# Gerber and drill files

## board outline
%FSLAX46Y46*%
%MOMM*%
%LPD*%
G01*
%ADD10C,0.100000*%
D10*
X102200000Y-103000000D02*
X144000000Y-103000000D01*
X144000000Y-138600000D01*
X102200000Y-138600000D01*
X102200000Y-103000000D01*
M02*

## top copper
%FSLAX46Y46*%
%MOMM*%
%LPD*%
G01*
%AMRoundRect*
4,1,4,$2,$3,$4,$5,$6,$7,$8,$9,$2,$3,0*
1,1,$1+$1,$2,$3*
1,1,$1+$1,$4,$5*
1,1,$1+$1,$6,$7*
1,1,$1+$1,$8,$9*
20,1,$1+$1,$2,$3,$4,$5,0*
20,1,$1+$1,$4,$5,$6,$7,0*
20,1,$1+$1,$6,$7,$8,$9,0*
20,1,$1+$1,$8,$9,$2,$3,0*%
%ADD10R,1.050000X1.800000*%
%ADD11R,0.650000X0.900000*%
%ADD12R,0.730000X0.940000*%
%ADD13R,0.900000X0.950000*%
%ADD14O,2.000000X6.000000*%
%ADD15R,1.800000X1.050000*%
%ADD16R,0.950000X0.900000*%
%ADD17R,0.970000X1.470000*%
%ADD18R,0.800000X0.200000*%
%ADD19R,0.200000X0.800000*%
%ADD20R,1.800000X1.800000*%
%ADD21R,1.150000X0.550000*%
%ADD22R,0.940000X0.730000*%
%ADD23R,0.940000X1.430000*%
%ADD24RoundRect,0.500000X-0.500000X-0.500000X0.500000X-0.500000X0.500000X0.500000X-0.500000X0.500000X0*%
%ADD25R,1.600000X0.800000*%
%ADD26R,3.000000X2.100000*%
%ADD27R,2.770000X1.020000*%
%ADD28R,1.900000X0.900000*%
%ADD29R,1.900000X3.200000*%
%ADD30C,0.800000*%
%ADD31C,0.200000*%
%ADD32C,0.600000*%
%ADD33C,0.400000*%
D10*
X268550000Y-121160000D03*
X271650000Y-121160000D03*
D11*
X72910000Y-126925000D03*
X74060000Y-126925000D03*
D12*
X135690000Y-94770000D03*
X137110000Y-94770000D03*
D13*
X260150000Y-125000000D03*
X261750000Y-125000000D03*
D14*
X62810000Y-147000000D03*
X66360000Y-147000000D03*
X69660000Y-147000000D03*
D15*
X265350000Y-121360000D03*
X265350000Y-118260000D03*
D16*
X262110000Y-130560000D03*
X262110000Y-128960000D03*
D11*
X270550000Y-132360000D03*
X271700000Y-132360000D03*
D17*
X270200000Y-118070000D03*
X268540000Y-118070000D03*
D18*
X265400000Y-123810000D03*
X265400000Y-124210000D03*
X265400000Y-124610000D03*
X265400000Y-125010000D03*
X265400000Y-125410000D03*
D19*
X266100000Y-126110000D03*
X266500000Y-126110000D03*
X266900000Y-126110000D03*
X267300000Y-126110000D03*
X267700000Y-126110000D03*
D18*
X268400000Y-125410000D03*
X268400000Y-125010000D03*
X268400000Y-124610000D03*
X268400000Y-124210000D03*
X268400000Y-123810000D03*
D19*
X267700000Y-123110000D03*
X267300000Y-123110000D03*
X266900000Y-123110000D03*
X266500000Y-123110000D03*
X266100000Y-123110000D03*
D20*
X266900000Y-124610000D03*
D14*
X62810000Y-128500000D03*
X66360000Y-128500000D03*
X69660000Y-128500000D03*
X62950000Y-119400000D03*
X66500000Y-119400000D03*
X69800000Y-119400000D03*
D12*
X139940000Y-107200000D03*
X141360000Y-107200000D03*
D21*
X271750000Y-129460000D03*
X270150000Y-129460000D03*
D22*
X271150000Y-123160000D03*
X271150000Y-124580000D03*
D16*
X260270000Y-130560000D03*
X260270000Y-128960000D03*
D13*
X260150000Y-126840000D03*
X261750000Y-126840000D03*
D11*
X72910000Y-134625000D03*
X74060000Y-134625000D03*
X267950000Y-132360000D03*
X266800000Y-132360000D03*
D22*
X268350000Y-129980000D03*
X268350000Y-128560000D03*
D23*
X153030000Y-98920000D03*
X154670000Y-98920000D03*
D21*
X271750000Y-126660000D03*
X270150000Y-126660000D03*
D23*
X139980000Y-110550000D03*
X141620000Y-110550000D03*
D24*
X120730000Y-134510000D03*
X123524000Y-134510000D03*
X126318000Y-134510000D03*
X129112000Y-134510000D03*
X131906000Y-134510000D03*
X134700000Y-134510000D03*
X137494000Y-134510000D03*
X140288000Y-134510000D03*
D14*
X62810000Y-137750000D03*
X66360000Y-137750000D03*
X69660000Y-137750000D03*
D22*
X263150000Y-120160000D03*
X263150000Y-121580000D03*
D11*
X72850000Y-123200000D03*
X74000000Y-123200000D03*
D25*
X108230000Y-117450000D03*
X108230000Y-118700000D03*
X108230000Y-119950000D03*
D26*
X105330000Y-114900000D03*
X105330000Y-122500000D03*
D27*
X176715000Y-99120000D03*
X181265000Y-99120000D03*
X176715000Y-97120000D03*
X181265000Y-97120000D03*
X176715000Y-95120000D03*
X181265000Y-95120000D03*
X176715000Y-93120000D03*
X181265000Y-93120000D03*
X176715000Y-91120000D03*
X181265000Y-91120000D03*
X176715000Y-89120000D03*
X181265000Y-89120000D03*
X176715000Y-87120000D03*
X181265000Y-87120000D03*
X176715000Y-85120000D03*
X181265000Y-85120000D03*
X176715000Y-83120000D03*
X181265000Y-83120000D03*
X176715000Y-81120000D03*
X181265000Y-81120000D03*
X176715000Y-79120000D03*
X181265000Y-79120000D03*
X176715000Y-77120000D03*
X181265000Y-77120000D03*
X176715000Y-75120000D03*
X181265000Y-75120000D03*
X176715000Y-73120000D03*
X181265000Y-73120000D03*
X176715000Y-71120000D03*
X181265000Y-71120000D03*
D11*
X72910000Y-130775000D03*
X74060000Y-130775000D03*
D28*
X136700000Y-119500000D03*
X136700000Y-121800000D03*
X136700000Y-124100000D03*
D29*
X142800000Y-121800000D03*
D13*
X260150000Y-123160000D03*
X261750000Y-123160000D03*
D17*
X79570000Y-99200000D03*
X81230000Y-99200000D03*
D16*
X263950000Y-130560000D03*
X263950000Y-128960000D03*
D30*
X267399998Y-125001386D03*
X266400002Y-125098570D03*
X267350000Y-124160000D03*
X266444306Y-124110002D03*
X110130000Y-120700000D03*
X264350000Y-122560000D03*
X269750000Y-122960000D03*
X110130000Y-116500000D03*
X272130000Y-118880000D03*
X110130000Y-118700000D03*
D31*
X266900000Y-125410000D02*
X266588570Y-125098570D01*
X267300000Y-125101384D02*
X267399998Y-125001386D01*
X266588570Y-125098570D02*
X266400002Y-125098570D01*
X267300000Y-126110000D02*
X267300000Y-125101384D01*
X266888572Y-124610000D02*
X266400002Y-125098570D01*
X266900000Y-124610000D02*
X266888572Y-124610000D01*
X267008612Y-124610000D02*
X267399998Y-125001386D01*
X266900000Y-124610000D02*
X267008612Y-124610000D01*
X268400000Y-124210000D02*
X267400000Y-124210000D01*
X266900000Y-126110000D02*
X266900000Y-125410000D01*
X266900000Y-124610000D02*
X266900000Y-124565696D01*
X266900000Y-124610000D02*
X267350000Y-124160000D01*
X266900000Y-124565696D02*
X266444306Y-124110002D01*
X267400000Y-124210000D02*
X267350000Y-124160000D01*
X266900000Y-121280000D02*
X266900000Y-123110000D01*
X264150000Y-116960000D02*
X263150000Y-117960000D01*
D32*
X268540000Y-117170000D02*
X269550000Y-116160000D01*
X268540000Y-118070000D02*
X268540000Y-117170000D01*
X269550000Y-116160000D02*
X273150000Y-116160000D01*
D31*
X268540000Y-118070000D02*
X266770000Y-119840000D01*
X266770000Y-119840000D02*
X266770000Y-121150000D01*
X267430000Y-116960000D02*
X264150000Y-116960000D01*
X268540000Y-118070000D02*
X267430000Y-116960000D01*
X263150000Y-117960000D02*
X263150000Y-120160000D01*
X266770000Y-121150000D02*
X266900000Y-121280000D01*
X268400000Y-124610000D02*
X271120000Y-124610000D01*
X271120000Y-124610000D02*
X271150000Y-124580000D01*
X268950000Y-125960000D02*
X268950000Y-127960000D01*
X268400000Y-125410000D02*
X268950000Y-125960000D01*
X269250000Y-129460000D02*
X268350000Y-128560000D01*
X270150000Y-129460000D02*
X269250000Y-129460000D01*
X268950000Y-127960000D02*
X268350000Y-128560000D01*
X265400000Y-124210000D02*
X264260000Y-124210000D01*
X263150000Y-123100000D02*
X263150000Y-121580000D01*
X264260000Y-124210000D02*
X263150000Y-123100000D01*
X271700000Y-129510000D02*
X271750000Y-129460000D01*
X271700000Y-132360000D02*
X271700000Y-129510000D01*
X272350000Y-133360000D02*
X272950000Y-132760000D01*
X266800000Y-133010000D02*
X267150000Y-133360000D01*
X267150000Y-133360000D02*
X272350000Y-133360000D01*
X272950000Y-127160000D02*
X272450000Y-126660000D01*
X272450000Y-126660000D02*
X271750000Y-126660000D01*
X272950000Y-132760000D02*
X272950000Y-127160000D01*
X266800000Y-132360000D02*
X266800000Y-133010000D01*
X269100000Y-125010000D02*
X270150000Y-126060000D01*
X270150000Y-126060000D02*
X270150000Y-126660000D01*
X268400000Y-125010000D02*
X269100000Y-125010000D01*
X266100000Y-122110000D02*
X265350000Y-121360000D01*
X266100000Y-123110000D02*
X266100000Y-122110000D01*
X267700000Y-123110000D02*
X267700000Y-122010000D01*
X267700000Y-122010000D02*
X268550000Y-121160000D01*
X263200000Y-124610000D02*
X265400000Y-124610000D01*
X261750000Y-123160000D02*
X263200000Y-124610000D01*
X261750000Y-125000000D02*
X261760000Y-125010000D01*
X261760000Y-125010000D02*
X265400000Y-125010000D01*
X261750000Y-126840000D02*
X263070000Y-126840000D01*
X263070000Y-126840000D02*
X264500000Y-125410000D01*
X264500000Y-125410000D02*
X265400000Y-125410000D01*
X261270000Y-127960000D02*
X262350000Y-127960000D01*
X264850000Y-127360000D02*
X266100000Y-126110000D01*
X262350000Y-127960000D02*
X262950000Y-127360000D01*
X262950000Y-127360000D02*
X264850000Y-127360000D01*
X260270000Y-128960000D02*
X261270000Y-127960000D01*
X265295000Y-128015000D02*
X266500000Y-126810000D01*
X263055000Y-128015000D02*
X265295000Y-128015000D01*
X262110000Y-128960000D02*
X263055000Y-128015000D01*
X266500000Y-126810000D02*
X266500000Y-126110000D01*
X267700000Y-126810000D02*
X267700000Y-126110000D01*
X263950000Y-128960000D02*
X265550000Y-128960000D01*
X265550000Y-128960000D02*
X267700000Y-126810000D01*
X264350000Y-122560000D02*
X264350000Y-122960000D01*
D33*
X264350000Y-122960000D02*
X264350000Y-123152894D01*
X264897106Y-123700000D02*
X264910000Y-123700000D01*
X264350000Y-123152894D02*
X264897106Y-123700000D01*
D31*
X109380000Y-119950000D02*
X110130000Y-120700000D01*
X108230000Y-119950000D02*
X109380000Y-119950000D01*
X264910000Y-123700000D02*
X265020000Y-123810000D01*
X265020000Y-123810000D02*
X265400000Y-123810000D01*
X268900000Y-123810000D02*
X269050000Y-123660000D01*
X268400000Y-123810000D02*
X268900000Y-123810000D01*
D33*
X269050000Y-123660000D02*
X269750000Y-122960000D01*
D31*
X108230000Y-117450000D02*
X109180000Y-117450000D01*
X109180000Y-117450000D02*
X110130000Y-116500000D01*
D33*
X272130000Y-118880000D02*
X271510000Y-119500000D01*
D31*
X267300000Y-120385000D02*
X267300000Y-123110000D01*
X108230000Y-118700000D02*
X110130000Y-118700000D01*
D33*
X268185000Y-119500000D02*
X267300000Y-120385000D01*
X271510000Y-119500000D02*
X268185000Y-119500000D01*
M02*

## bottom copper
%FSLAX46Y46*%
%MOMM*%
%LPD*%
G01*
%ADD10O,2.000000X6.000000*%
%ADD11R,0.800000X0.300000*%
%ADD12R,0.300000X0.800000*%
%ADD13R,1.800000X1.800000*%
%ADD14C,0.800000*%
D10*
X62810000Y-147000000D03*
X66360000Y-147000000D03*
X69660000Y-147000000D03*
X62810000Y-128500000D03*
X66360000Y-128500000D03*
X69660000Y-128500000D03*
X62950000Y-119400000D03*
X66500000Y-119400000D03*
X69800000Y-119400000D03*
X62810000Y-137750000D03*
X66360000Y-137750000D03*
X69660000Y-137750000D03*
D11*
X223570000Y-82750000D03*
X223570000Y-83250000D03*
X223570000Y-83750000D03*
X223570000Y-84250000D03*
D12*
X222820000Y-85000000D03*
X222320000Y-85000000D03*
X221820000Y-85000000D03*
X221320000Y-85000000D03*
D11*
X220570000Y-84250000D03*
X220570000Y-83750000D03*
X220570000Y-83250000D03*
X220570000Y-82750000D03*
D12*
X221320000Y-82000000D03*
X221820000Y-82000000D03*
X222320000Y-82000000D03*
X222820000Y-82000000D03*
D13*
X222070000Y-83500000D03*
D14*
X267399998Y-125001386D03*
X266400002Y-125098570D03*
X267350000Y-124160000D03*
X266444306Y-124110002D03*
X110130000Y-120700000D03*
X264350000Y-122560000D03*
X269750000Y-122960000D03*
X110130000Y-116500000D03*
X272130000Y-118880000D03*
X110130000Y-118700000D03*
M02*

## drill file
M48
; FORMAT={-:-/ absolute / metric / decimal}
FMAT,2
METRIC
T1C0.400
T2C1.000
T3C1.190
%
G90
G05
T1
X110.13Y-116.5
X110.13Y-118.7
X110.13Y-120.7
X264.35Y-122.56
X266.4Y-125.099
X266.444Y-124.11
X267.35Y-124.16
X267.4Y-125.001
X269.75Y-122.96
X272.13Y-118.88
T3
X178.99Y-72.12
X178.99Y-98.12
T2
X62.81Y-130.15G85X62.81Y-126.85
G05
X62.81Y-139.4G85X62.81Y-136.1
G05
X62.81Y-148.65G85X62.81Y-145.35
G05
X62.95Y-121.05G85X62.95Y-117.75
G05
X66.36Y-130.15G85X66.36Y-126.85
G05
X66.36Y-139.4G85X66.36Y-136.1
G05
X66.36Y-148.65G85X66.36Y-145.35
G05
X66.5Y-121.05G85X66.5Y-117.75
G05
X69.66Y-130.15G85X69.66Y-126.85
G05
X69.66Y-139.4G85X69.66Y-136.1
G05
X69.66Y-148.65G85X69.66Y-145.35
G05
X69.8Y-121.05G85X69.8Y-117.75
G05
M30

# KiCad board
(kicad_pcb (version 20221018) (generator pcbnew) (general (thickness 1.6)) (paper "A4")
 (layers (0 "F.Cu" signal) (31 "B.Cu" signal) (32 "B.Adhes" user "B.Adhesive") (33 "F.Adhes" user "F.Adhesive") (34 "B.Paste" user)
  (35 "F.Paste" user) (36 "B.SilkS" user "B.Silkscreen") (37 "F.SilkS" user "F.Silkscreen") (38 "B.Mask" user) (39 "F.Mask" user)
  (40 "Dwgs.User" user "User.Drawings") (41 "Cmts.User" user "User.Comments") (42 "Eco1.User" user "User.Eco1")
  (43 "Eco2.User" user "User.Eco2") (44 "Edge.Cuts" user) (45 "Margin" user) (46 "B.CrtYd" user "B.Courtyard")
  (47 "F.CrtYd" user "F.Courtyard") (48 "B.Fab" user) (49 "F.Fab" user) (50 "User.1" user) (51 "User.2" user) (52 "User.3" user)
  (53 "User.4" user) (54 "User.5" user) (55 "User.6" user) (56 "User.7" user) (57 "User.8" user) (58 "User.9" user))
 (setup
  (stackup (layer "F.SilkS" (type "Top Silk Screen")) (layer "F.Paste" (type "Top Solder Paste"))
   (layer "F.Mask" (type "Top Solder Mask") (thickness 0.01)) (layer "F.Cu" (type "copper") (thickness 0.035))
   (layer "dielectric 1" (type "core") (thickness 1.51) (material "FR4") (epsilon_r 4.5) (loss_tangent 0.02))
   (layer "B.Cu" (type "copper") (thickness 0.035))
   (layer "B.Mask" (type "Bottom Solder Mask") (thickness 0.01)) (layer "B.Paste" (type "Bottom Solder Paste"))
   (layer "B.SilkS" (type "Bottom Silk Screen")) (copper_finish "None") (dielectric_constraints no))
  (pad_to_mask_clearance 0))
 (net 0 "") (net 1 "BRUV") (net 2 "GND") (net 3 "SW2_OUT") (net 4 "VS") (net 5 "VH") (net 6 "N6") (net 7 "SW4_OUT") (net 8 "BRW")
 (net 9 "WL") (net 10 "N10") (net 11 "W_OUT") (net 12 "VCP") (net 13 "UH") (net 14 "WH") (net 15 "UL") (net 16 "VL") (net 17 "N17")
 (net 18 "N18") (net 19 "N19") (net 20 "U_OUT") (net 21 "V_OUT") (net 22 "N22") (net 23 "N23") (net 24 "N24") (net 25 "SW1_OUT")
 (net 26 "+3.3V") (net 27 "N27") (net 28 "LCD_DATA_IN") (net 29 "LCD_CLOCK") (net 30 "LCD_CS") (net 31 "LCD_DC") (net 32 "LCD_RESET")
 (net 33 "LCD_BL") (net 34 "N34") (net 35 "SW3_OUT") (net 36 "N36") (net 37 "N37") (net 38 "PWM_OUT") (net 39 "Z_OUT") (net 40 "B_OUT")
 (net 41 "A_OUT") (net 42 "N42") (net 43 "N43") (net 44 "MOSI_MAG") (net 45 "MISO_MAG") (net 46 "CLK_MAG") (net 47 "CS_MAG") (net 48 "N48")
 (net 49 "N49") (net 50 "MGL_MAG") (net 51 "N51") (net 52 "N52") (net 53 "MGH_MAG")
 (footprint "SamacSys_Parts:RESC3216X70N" (layer "F.Cu") (at 270.1 121.16)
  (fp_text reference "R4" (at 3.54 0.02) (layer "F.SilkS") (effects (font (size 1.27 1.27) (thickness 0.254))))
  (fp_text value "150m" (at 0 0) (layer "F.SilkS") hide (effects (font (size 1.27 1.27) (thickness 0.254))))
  (pad "1" smd rect (at -1.55 0) (size 1.05 1.8) (layers "F.Cu" "F.Paste" "F.Mask") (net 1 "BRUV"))
  (pad "2" smd rect (at 1.55 0) (size 1.05 1.8) (layers "F.Cu" "F.Paste" "F.Mask") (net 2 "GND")))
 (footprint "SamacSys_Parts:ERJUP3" (layer "F.Cu") (at 73.485 126.925)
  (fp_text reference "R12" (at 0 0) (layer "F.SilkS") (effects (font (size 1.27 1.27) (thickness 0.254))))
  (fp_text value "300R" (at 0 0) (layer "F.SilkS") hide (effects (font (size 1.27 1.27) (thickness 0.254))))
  (pad "1" smd rect (at -0.575 0) (size 0.65 0.9) (layers "F.Cu" "F.Paste" "F.Mask") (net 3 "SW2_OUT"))
  (pad "2" smd rect (at 0.575 0) (size 0.65 0.9) (layers "F.Cu" "F.Paste" "F.Mask") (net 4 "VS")))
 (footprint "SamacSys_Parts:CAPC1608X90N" (layer "F.Cu") (at 136.4 94.77)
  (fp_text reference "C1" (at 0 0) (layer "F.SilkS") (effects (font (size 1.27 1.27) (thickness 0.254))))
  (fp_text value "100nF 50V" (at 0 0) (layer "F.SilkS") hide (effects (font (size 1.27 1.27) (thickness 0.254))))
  (pad "1" smd rect (at -0.71 0) (size 0.73 0.94) (layers "F.Cu" "F.Paste" "F.Mask") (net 2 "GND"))
  (pad "2" smd rect (at 0.71 0) (size 0.73 0.94) (layers "F.Cu" "F.Paste" "F.Mask") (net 4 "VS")))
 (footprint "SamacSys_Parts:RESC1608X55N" (layer "F.Cu") (at 260.95 125)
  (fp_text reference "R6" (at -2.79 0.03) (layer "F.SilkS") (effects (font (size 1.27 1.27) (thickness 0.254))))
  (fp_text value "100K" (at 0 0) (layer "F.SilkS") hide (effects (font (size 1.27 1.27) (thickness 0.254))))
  (pad "1" smd rect (at -0.8 0) (size 0.9 0.95) (layers "F.Cu" "F.Paste" "F.Mask") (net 2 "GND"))
  (pad "2" smd rect (at 0.8 0) (size 0.9 0.95) (layers "F.Cu" "F.Paste" "F.Mask") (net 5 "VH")))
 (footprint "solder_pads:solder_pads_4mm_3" (layer "F.Cu") (at 66.6 152)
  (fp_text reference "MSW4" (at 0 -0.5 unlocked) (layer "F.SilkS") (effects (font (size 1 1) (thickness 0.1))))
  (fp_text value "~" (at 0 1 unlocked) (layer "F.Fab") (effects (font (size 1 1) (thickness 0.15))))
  (pad "1" thru_hole oval (at -3.79 -5 90) (size 6 2) (drill oval 4.3 1) (layers "*.Cu" "*.Mask") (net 2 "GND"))
  (pad "2" thru_hole oval (at -0.24 -5 90) (size 6 2) (drill oval 4.3 1) (layers "*.Cu" "*.Mask") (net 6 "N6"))
  (pad "4" thru_hole oval (at 3.06 -5 90) (size 6 2) (drill oval 4.3 1) (layers "*.Cu" "*.Mask") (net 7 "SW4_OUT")))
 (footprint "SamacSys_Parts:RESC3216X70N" (layer "F.Cu") (at 265.35 119.81 90)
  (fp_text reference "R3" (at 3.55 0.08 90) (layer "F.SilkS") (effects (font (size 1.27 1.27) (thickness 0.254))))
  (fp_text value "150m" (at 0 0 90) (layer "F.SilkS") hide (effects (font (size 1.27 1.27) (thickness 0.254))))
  (pad "1" smd rect (at -1.55 0 90) (size 1.05 1.8) (layers "F.Cu" "F.Paste" "F.Mask") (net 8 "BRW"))
  (pad "2" smd rect (at 1.55 0 90) (size 1.05 1.8) (layers "F.Cu" "F.Paste" "F.Mask") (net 2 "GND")))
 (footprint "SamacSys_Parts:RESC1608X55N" (layer "F.Cu") (at 262.11 129.76 90)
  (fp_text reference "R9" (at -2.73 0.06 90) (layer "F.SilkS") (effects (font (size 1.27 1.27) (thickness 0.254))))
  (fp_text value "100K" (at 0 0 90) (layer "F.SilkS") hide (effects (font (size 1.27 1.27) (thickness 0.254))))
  (pad "1" smd rect (at -0.8 0 90) (size 0.9 0.95) (layers "F.Cu" "F.Paste" "F.Mask") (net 2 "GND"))
  (pad "2" smd rect (at 0.8 0 90) (size 0.9 0.95) (layers "F.Cu" "F.Paste" "F.Mask") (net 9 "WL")))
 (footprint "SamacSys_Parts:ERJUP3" (layer "F.Cu") (at 271.125 132.36)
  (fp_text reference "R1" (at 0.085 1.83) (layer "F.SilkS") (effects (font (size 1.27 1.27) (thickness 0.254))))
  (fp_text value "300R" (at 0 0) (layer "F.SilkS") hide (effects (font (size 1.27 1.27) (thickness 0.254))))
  (pad "1" smd rect (at -0.575 0) (size 0.65 0.9) (layers "F.Cu" "F.Paste" "F.Mask") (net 2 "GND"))
  (pad "2" smd rect (at 0.575 0) (size 0.65 0.9) (layers "F.Cu" "F.Paste" "F.Mask") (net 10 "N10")))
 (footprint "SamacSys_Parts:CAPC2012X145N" (layer "F.Cu") (at 269.37 118.07 180)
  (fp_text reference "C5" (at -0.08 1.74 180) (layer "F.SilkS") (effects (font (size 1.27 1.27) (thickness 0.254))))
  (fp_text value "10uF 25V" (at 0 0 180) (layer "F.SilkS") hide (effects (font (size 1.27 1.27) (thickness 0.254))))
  (pad "1" smd rect (at -0.83 0 180) (size 0.97 1.47) (layers "F.Cu" "F.Paste" "F.Mask") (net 2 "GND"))
  (pad "2" smd rect (at 0.83 0 180) (size 0.97 1.47) (layers "F.Cu" "F.Paste" "F.Mask") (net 4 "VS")))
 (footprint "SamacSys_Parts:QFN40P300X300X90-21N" (layer "F.Cu") (at 266.9 124.61)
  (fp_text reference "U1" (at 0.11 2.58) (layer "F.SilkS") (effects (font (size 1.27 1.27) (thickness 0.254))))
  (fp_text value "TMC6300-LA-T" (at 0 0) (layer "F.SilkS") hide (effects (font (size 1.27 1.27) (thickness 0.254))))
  (pad "1" smd rect (at -1.5 -0.8 90) (size 0.2 0.8) (layers "F.Cu" "F.Paste" "F.Mask") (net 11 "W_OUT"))
  (pad "2" smd rect (at -1.5 -0.4 90) (size 0.2 0.8) (layers "F.Cu" "F.Paste" "F.Mask") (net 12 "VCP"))
  (pad "3" smd rect (at -1.5 0 90) (size 0.2 0.8) (layers "F.Cu" "F.Paste" "F.Mask") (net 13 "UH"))
  (pad "4" smd rect (at -1.5 0.4 90) (size 0.2 0.8) (layers "F.Cu" "F.Paste" "F.Mask") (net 5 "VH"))
  (pad "5" smd rect (at -1.5 0.8 90) (size 0.2 0.8) (layers "F.Cu" "F.Paste" "F.Mask") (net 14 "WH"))
  (pad "6" smd rect (at -0.8 1.5) (size 0.2 0.8) (layers "F.Cu" "F.Paste" "F.Mask") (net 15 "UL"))
  (pad "7" smd rect (at -0.4 1.5) (size 0.2 0.8) (layers "F.Cu" "F.Paste" "F.Mask") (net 9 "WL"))
  (pad "8" smd rect (at 0 1.5) (size 0.2 0.8) (layers "F.Cu" "F.Paste" "F.Mask") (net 2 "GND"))
  (pad "9" smd rect (at 0.4 1.5) (size 0.2 0.8) (layers "F.Cu" "F.Paste" "F.Mask") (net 2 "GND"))
  (pad "10" smd rect (at 0.8 1.5) (size 0.2 0.8) (layers "F.Cu" "F.Paste" "F.Mask") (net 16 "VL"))
  (pad "11" smd rect (at 1.5 0.8 90) (size 0.2 0.8) (layers "F.Cu" "F.Paste" "F.Mask") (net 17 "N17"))
  (pad "12" smd rect (at 1.5 0.4 90) (size 0.2 0.8) (layers "F.Cu" "F.Paste" "F.Mask") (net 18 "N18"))
  (pad "13" smd rect (at 1.5 0 90) (size 0.2 0.8) (layers "F.Cu" "F.Paste" "F.Mask") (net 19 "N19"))
  (pad "14" smd rect (at 1.5 -0.4 90) (size 0.2 0.8) (layers "F.Cu" "F.Paste" "F.Mask") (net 2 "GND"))
  (pad "15" smd rect (at 1.5 -0.8 90) (size 0.2 0.8) (layers "F.Cu" "F.Paste" "F.Mask") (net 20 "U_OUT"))
  (pad "16" smd rect (at 0.8 -1.5) (size 0.2 0.8) (layers "F.Cu" "F.Paste" "F.Mask") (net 1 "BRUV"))
  (pad "17" smd rect (at 0.4 -1.5) (size 0.2 0.8) (layers "F.Cu" "F.Paste" "F.Mask") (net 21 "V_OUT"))
  (pad "18" smd rect (at 0 -1.5) (size 0.2 0.8) (layers "F.Cu" "F.Paste" "F.Mask") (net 4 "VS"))
  (pad "19" smd rect (at -0.4 -1.5) (size 0.2 0.8) (layers "F.Cu" "F.Paste" "F.Mask") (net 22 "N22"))
  (pad "20" smd rect (at -0.8 -1.5) (size 0.2 0.8) (layers "F.Cu" "F.Paste" "F.Mask") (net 8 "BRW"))
  (pad "21" smd rect (at 0 0) (size 1.8 1.8) (layers "F.Cu" "F.Paste" "F.Mask") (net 2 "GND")))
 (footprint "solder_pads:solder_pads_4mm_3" (layer "F.Cu") (at 66.6 133.5)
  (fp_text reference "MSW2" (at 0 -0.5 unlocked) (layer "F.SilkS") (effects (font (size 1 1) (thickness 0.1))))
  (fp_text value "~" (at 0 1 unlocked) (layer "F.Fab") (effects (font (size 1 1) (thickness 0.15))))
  (pad "1" thru_hole oval (at -3.79 -5 90) (size 6 2) (drill oval 4.3 1) (layers "*.Cu" "*.Mask") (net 2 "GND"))
  (pad "2" thru_hole oval (at -0.24 -5 90) (size 6 2) (drill oval 4.3 1) (layers "*.Cu" "*.Mask") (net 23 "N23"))
  (pad "4" thru_hole oval (at 3.06 -5 90) (size 6 2) (drill oval 4.3 1) (layers "*.Cu" "*.Mask") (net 3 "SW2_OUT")))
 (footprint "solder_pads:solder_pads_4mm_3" (layer "F.Cu") (at 66.74 124.4)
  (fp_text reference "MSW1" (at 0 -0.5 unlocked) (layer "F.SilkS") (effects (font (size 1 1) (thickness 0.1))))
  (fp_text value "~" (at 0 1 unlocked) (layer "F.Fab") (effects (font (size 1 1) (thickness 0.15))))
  (pad "1" thru_hole oval (at -3.79 -5 90) (size 6 2) (drill oval 4.3 1) (layers "*.Cu" "*.Mask") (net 2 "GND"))
  (pad "2" thru_hole oval (at -0.24 -5 90) (size 6 2) (drill oval 4.3 1) (layers "*.Cu" "*.Mask") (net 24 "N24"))
  (pad "4" thru_hole oval (at 3.06 -5 90) (size 6 2) (drill oval 4.3 1) (layers "*.Cu" "*.Mask") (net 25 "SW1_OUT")))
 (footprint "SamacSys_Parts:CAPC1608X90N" (layer "F.Cu") (at 140.65 107.2)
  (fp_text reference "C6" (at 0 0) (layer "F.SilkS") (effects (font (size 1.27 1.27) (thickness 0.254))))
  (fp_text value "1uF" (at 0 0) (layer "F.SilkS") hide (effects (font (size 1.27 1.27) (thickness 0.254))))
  (pad "1" smd rect (at -0.71 0) (size 0.73 0.94) (layers "F.Cu" "F.Paste" "F.Mask") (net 2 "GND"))
  (pad "2" smd rect (at 0.71 0) (size 0.73 0.94) (layers "F.Cu" "F.Paste" "F.Mask") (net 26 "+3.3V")))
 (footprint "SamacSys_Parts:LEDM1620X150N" (layer "F.Cu") (at 270.95 129.46 180)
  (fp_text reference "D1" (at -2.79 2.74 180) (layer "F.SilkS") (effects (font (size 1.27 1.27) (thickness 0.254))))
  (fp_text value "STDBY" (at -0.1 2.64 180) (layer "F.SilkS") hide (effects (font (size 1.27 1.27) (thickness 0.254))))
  (pad "1" smd rect (at -0.8 0 270) (size 0.55 1.15) (layers "F.Cu" "F.Paste" "F.Mask") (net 10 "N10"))
  (pad "2" smd rect (at 0.8 0 270) (size 0.55 1.15) (layers "F.Cu" "F.Paste" "F.Mask") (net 17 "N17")))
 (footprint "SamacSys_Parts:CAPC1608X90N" (layer "F.Cu") (at 271.15 123.87 -90)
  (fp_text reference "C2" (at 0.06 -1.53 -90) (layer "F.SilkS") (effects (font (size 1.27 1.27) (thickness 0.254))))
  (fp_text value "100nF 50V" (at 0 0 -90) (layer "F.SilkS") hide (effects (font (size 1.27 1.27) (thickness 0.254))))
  (pad "1" smd rect (at -0.71 0 270) (size 0.73 0.94) (layers "F.Cu" "F.Paste" "F.Mask") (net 2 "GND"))
  (pad "2" smd rect (at 0.71 0 270) (size 0.73 0.94) (layers "F.Cu" "F.Paste" "F.Mask") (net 19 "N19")))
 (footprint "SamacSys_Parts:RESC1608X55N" (layer "F.Cu") (at 260.27 129.76 90)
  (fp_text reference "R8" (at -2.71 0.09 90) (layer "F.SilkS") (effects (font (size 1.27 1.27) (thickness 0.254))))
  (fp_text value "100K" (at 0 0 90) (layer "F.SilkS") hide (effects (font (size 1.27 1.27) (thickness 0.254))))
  (pad "1" smd rect (at -0.8 0 90) (size 0.9 0.95) (layers "F.Cu" "F.Paste" "F.Mask") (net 2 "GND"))
  (pad "2" smd rect (at 0.8 0 90) (size 0.9 0.95) (layers "F.Cu" "F.Paste" "F.Mask") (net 15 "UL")))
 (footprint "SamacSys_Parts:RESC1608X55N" (layer "F.Cu") (at 260.95 126.84)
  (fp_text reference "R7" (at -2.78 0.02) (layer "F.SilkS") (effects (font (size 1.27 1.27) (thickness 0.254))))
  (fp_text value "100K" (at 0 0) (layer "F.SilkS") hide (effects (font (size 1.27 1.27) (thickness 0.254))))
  (pad "1" smd rect (at -0.8 0) (size 0.9 0.95) (layers "F.Cu" "F.Paste" "F.Mask") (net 2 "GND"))
  (pad "2" smd rect (at 0.8 0) (size 0.9 0.95) (layers "F.Cu" "F.Paste" "F.Mask") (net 14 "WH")))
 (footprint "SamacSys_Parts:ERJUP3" (layer "F.Cu") (at 73.485 134.625)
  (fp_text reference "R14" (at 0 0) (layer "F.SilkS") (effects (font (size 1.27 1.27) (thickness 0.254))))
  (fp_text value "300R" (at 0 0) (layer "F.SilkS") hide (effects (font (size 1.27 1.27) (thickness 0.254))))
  (pad "1" smd rect (at -0.575 0) (size 0.65 0.9) (layers "F.Cu" "F.Paste" "F.Mask") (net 7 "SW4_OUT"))
  (pad "2" smd rect (at 0.575 0) (size 0.65 0.9) (layers "F.Cu" "F.Paste" "F.Mask") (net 4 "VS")))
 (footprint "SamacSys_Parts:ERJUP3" (layer "F.Cu") (at 267.375 132.36 180)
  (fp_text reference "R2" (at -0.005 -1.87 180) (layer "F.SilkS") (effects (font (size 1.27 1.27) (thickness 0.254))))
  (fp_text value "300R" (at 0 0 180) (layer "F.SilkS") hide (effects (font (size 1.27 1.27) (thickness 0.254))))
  (pad "1" smd rect (at -0.575 0 180) (size 0.65 0.9) (layers "F.Cu" "F.Paste" "F.Mask") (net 2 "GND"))
  (pad "2" smd rect (at 0.575 0 180) (size 0.65 0.9) (layers "F.Cu" "F.Paste" "F.Mask") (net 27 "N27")))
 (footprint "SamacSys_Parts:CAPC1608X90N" (layer "F.Cu") (at 268.35 129.27 90)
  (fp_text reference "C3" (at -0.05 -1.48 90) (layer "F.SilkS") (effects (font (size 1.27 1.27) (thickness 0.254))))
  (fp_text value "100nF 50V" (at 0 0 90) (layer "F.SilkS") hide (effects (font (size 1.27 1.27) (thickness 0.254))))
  (pad "1" smd rect (at -0.71 0 90) (size 0.73 0.94) (layers "F.Cu" "F.Paste" "F.Mask") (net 2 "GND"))
  (pad "2" smd rect (at 0.71 0 90) (size 0.73 0.94) (layers "F.Cu" "F.Paste" "F.Mask") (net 17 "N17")))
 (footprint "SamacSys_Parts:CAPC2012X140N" (layer "F.Cu") (at 153.85 98.92)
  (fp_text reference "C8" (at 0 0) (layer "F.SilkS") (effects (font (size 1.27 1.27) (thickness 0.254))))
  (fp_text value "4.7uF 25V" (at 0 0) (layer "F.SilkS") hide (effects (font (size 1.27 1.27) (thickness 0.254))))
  (pad "1" smd rect (at -0.82 0) (size 0.94 1.43) (layers "F.Cu" "F.Paste" "F.Mask") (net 2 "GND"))
  (pad "2" smd rect (at 0.82 0) (size 0.94 1.43) (layers "F.Cu" "F.Paste" "F.Mask") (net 4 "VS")))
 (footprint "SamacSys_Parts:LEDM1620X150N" (layer "F.Cu") (at 270.95 126.66 180)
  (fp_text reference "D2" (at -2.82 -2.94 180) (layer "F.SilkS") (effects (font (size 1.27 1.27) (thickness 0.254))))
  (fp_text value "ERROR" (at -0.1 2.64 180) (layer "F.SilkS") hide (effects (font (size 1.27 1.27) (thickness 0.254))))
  (pad "1" smd rect (at -0.8 0 270) (size 0.55 1.15) (layers "F.Cu" "F.Paste" "F.Mask") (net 27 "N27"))
  (pad "2" smd rect (at 0.8 0 270) (size 0.55 1.15) (layers "F.Cu" "F.Paste" "F.Mask") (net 18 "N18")))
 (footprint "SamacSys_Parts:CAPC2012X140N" (layer "F.Cu") (at 140.8 110.55)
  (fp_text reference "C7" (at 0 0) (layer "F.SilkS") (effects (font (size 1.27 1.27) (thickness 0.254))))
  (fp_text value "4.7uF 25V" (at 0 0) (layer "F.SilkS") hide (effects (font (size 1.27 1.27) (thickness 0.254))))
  (pad "1" smd rect (at -0.82 0) (size 0.94 1.43) (layers "F.Cu" "F.Paste" "F.Mask") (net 2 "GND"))
  (pad "2" smd rect (at 0.82 0) (size 0.94 1.43) (layers "F.Cu" "F.Paste" "F.Mask") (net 26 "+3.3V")))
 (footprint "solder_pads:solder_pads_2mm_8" (layer "F.Cu") (at 130.128 137.05)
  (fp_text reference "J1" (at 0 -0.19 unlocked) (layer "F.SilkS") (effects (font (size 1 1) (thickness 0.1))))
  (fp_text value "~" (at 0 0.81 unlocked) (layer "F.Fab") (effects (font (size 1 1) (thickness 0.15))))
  (pad "1" smd roundrect (at -9.398 -2.54) (size 2 2) (layers "F.Cu" "F.Paste" "F.Mask") (roundrect_rratio 0.25) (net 26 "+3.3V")
   (thermal_bridge_angle 45))
  (pad "2" smd roundrect (at -6.604 -2.54) (size 2 2) (layers "F.Cu" "F.Paste" "F.Mask") (roundrect_rratio 0.25) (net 2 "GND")
   (thermal_bridge_angle 45))
  (pad "3" smd roundrect (at -3.81 -2.54) (size 2 2) (layers "F.Cu" "F.Paste" "F.Mask") (roundrect_rratio 0.25) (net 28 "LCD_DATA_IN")
   (thermal_bridge_angle 45))
  (pad "4" smd roundrect (at -1.016 -2.54) (size 2 2) (layers "F.Cu" "F.Paste" "F.Mask") (roundrect_rratio 0.25) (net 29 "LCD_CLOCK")
   (thermal_bridge_angle 45))
  (pad "5" smd roundrect (at 1.778 -2.54) (size 2 2) (layers "F.Cu" "F.Paste" "F.Mask") (roundrect_rratio 0.25) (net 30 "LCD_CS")
   (thermal_bridge_angle 45))
  (pad "6" smd roundrect (at 4.572 -2.54) (size 2 2) (layers "F.Cu" "F.Paste" "F.Mask") (roundrect_rratio 0.25) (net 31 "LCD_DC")
   (thermal_bridge_angle 45))
  (pad "7" smd roundrect (at 7.366 -2.54) (size 2 2) (layers "F.Cu" "F.Paste" "F.Mask") (roundrect_rratio 0.25) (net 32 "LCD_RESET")
   (thermal_bridge_angle 45))
  (pad "8" smd roundrect (at 10.16 -2.54) (size 2 2) (layers "F.Cu" "F.Paste" "F.Mask") (roundrect_rratio 0.25) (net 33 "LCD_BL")
   (thermal_bridge_angle 45)))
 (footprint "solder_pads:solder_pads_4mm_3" (layer "F.Cu") (at 66.6 142.75)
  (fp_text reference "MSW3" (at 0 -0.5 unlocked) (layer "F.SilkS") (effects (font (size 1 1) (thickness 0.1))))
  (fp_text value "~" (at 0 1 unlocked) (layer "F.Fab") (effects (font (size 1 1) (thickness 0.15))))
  (pad "1" thru_hole oval (at -3.79 -5 90) (size 6 2) (drill oval 4.3 1) (layers "*.Cu" "*.Mask") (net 2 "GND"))
  (pad "2" thru_hole oval (at -0.24 -5 90) (size 6 2) (drill oval 4.3 1) (layers "*.Cu" "*.Mask") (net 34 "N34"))
  (pad "4" thru_hole oval (at 3.06 -5 90) (size 6 2) (drill oval 4.3 1) (layers "*.Cu" "*.Mask") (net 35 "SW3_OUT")))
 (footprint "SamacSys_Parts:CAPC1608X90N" (layer "F.Cu") (at 263.15 120.87 -90)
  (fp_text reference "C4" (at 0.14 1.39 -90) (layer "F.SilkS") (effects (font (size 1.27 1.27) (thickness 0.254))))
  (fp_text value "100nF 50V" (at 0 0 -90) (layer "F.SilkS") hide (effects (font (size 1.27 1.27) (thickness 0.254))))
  (pad "1" smd rect (at -0.71 0 270) (size 0.73 0.94) (layers "F.Cu" "F.Paste" "F.Mask") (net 4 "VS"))
  (pad "2" smd rect (at 0.71 0 270) (size 0.73 0.94) (layers "F.Cu" "F.Paste" "F.Mask") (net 12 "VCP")))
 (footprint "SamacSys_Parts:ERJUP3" (layer "F.Cu") (at 73.425 123.2)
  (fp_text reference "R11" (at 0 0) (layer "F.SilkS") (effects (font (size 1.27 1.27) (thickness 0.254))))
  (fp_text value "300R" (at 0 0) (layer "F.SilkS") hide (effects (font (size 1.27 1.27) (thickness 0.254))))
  (pad "1" smd rect (at -0.575 0) (size 0.65 0.9) (layers "F.Cu" "F.Paste" "F.Mask") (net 25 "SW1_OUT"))
  (pad "2" smd rect (at 0.575 0) (size 0.65 0.9) (layers "F.Cu" "F.Paste" "F.Mask") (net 4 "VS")))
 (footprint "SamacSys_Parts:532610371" (layer "F.Cu") (at 105.33 118.7 -90)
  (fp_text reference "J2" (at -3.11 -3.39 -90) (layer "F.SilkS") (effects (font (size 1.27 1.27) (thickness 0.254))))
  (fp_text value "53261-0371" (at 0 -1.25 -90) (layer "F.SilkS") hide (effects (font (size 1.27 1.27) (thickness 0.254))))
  (pad "1" smd rect (at -1.25 -2.9 270) (size 0.8 1.6) (layers "F.Cu" "F.Paste" "F.Mask") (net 20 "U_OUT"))
  (pad "2" smd rect (at 0 -2.9 270) (size 0.8 1.6) (layers "F.Cu" "F.Paste" "F.Mask") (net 21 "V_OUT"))
  (pad "3" smd rect (at 1.25 -2.9 270) (size 0.8 1.6) (layers "F.Cu" "F.Paste" "F.Mask") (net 11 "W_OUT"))
  (pad "MP1" smd rect (at -3.8 0 270) (size 2.1 3) (layers "F.Cu" "F.Paste" "F.Mask") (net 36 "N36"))
  (pad "MP2" smd rect (at 3.8 0 270) (size 2.1 3) (layers "F.Cu" "F.Paste" "F.Mask") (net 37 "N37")))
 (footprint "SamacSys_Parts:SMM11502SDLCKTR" (layer "F.Cu") (at 178.99 85.12 -90)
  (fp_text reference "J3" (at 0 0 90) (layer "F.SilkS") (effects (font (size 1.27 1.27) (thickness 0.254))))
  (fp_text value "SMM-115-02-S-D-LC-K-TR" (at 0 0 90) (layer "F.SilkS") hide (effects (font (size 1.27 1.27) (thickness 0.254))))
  (pad "" np_thru_hole circle (at -13 0 270) (size 1.19 1.19) (drill 1.19) (layers "*.Cu" "*.Mask"))
  (pad "" np_thru_hole circle (at 13 0 270) (size 1.19 1.19) (drill 1.19) (layers "*.Cu" "*.Mask"))
  (pad "1" smd rect (at 14 2.275 270) (size 1.02 2.77) (layers "F.Cu" "F.Paste" "F.Mask") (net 33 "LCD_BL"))
  (pad "2" smd rect (at 14 -2.275 270) (size 1.02 2.77) (layers "F.Cu" "F.Paste" "F.Mask") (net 7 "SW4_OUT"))
  (pad "3" smd rect (at 12 2.275 270) (size 1.02 2.77) (layers "F.Cu" "F.Paste" "F.Mask") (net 32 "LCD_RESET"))
  (pad "4" smd rect (at 12 -2.275 270) (size 1.02 2.77) (layers "F.Cu" "F.Paste" "F.Mask") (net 35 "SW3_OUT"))
  (pad "5" smd rect (at 10 2.275 270) (size 1.02 2.77) (layers "F.Cu" "F.Paste" "F.Mask") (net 31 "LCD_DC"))
  (pad "6" smd rect (at 10 -2.275 270) (size 1.02 2.77) (layers "F.Cu" "F.Paste" "F.Mask") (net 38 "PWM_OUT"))
  (pad "7" smd rect (at 8 2.275 270) (size 1.02 2.77) (layers "F.Cu" "F.Paste" "F.Mask") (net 30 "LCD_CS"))
  (pad "8" smd rect (at 8 -2.275 270) (size 1.02 2.77) (layers "F.Cu" "F.Paste" "F.Mask") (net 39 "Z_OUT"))
  (pad "9" smd rect (at 6 2.275 270) (size 1.02 2.77) (layers "F.Cu" "F.Paste" "F.Mask") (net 29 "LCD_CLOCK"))
  (pad "10" smd rect (at 6 -2.275 270) (size 1.02 2.77) (layers "F.Cu" "F.Paste" "F.Mask") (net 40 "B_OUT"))
  (pad "11" smd rect (at 4 2.275 270) (size 1.02 2.77) (layers "F.Cu" "F.Paste" "F.Mask") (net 28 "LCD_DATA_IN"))
  (pad "12" smd rect (at 4 -2.275 270) (size 1.02 2.77) (layers "F.Cu" "F.Paste" "F.Mask") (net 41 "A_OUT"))
  (pad "13" smd rect (at 2 2.275 270) (size 1.02 2.77) (layers "F.Cu" "F.Paste" "F.Mask") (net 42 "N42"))
  (pad "14" smd rect (at 2 -2.275 270) (size 1.02 2.77) (layers "F.Cu" "F.Paste" "F.Mask") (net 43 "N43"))
  (pad "15" smd rect (at 0 2.275 270) (size 1.02 2.77) (layers "F.Cu" "F.Paste" "F.Mask") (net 3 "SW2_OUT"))
  (pad "16" smd rect (at 0 -2.275 270) (size 1.02 2.77) (layers "F.Cu" "F.Paste" "F.Mask") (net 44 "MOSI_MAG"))
  (pad "17" smd rect (at -2 2.275 270) (size 1.02 2.77) (layers "F.Cu" "F.Paste" "F.Mask") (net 25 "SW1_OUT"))
  (pad "18" smd rect (at -2 -2.275 270) (size 1.02 2.77) (layers "F.Cu" "F.Paste" "F.Mask") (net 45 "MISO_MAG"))
  (pad "19" smd rect (at -4 2.275 270) (size 1.02 2.77) (layers "F.Cu" "F.Paste" "F.Mask") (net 9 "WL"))
  (pad "20" smd rect (at -4 -2.275 270) (size 1.02 2.77) (layers "F.Cu" "F.Paste" "F.Mask") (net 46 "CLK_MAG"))
  (pad "21" smd rect (at -6 2.275 270) (size 1.02 2.77) (layers "F.Cu" "F.Paste" "F.Mask") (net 16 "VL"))
  (pad "22" smd rect (at -6 -2.275 270) (size 1.02 2.77) (layers "F.Cu" "F.Paste" "F.Mask") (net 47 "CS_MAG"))
  (pad "23" smd rect (at -8 2.275 270) (size 1.02 2.77) (layers "F.Cu" "F.Paste" "F.Mask") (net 15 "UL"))
  (pad "24" smd rect (at -8 -2.275 270) (size 1.02 2.77) (layers "F.Cu" "F.Paste" "F.Mask") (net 2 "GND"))
  (pad "25" smd rect (at -10 2.275 270) (size 1.02 2.77) (layers "F.Cu" "F.Paste" "F.Mask") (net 14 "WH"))
  (pad "26" smd rect (at -10 -2.275 270) (size 1.02 2.77) (layers "F.Cu" "F.Paste" "F.Mask") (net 2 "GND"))
  (pad "27" smd rect (at -12 2.275 270) (size 1.02 2.77) (layers "F.Cu" "F.Paste" "F.Mask") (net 5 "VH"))
  (pad "28" smd rect (at -12 -2.275 270) (size 1.02 2.77) (layers "F.Cu" "F.Paste" "F.Mask") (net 4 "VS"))
  (pad "29" smd rect (at -14 2.275 270) (size 1.02 2.77) (layers "F.Cu" "F.Paste" "F.Mask") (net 13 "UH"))
  (pad "30" smd rect (at -14 -2.275 270) (size 1.02 2.77) (layers "F.Cu" "F.Paste" "F.Mask") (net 4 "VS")))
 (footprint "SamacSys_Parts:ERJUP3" (layer "F.Cu") (at 73.485 130.775)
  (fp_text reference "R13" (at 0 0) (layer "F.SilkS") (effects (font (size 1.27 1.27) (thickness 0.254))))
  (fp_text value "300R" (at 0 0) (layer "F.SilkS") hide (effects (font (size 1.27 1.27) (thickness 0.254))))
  (pad "1" smd rect (at -0.575 0) (size 0.65 0.9) (layers "F.Cu" "F.Paste" "F.Mask") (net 35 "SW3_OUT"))
  (pad "2" smd rect (at 0.575 0) (size 0.65 0.9) (layers "F.Cu" "F.Paste" "F.Mask") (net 4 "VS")))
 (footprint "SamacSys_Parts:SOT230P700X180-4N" (layer "F.Cu") (at 139.75 121.8)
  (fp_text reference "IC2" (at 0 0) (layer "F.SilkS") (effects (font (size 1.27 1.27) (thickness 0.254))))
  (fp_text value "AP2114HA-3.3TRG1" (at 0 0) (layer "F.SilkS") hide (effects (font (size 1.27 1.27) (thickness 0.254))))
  (pad "1" smd rect (at -3.05 -2.3 90) (size 0.9 1.9) (layers "F.Cu" "F.Paste" "F.Mask") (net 4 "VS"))
  (pad "2" smd rect (at -3.05 0 90) (size 0.9 1.9) (layers "F.Cu" "F.Paste" "F.Mask") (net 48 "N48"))
  (pad "3" smd rect (at -3.05 2.3 90) (size 0.9 1.9) (layers "F.Cu" "F.Paste" "F.Mask") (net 26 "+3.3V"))
  (pad "4" smd rect (at 3.05 0) (size 1.9 3.2) (layers "F.Cu" "F.Paste" "F.Mask") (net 2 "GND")))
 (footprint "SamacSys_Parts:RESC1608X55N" (layer "F.Cu") (at 260.95 123.16)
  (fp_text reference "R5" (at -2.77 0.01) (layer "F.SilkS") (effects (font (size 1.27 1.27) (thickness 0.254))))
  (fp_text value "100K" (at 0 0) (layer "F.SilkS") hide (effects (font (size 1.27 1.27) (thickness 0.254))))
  (pad "1" smd rect (at -0.8 0) (size 0.9 0.95) (layers "F.Cu" "F.Paste" "F.Mask") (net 2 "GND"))
  (pad "2" smd rect (at 0.8 0) (size 0.9 0.95) (layers "F.Cu" "F.Paste" "F.Mask") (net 13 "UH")))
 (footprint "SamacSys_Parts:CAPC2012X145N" (layer "F.Cu") (at 80.4 99.2)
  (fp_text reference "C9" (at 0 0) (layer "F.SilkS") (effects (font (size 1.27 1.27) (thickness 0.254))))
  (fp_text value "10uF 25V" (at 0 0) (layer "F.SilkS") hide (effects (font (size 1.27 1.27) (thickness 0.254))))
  (pad "1" smd rect (at -0.83 0) (size 0.97 1.47) (layers "F.Cu" "F.Paste" "F.Mask") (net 2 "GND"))
  (pad "2" smd rect (at 0.83 0) (size 0.97 1.47) (layers "F.Cu" "F.Paste" "F.Mask") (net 26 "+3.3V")))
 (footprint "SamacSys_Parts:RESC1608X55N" (layer "F.Cu") (at 263.95 129.76 90)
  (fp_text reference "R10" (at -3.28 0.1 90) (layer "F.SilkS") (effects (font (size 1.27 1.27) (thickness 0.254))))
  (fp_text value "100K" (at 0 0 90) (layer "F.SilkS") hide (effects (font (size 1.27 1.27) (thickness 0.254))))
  (pad "1" smd rect (at -0.8 0 90) (size 0.9 0.95) (layers "F.Cu" "F.Paste" "F.Mask") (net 2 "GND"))
  (pad "2" smd rect (at 0.8 0 90) (size 0.9 0.95) (layers "F.Cu" "F.Paste" "F.Mask") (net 16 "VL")))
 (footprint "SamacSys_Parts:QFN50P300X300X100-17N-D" (layer "B.Cu") (at 222.07 83.5 180)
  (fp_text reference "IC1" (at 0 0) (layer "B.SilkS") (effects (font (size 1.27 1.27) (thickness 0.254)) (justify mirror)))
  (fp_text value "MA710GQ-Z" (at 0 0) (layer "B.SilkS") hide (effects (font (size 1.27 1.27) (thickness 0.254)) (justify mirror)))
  (pad "1" smd rect (at -1.5 0.75 90) (size 0.3 0.8) (layers "B.Cu" "B.Paste" "B.Mask") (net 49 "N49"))
  (pad "2" smd rect (at -1.5 0.25 90) (size 0.3 0.8) (layers "B.Cu" "B.Paste" "B.Mask") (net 41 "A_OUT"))
  (pad "3" smd rect (at -1.5 -0.25 90) (size 0.3 0.8) (layers "B.Cu" "B.Paste" "B.Mask") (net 39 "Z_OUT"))
  (pad "4" smd rect (at -1.5 -0.75 90) (size 0.3 0.8) (layers "B.Cu" "B.Paste" "B.Mask") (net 44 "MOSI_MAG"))
  (pad "5" smd rect (at -0.75 -1.5 180) (size 0.3 0.8) (layers "B.Cu" "B.Paste" "B.Mask") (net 47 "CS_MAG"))
  (pad "6" smd rect (at -0.25 -1.5 180) (size 0.3 0.8) (layers "B.Cu" "B.Paste" "B.Mask") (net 40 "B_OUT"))
  (pad "7" smd rect (at 0.25 -1.5 180) (size 0.3 0.8) (layers "B.Cu" "B.Paste" "B.Mask") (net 45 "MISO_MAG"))
  (pad "8" smd rect (at 0.75 -1.5 180) (size 0.3 0.8) (layers "B.Cu" "B.Paste" "B.Mask") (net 2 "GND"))
  (pad "9" smd rect (at 1.5 -0.75 90) (size 0.3 0.8) (layers "B.Cu" "B.Paste" "B.Mask") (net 38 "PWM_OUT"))
  (pad "10" smd rect (at 1.5 -0.25 90) (size 0.3 0.8) (layers "B.Cu" "B.Paste" "B.Mask") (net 2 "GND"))
  (pad "11" smd rect (at 1.5 0.25 90) (size 0.3 0.8) (layers "B.Cu" "B.Paste" "B.Mask") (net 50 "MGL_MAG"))
  (pad "12" smd rect (at 1.5 0.75 90) (size 0.3 0.8) (layers "B.Cu" "B.Paste" "B.Mask") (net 46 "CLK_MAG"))
  (pad "13" smd rect (at 0.75 1.5 180) (size 0.3 0.8) (layers "B.Cu" "B.Paste" "B.Mask") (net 26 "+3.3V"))
  (pad "14" smd rect (at 0.25 1.5 180) (size 0.3 0.8) (layers "B.Cu" "B.Paste" "B.Mask") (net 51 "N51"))
  (pad "15" smd rect (at -0.25 1.5 180) (size 0.3 0.8) (layers "B.Cu" "B.Paste" "B.Mask") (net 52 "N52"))
  (pad "16" smd rect (at -0.75 1.5 180) (size 0.3 0.8) (layers "B.Cu" "B.Paste" "B.Mask") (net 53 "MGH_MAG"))
  (pad "17" smd rect (at 0 0 180) (size 1.8 1.8) (layers "B.Cu" "B.Paste" "B.Mask") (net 2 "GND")))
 (gr_rect (start 102.2 103) (end 144 138.6) (stroke (width 0.1) (type default)) (fill none) (layer "Edge.Cuts"))
 (segment (start 266.9 125.41) (end 266.58857 125.09857) (width 0.2) (layer "F.Cu") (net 2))
 (segment (start 267.3 125.101384) (end 267.399998 125.001386) (width 0.2) (layer "F.Cu") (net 2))
 (segment (start 266.58857 125.09857) (end 266.400002 125.09857) (width 0.2) (layer "F.Cu") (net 2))
 (segment (start 267.3 126.11) (end 267.3 125.101384) (width 0.2) (layer "F.Cu") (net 2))
 (segment (start 266.888572 124.61) (end 266.400002 125.09857) (width 0.2) (layer "F.Cu") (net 2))
 (segment (start 266.9 124.61) (end 266.888572 124.61) (width 0.2) (layer "F.Cu") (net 2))
 (segment (start 267.008612 124.61) (end 267.399998 125.001386) (width 0.2) (layer "F.Cu") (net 2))
 (segment (start 266.9 124.61) (end 267.008612 124.61) (width 0.2) (layer "F.Cu") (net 2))
 (segment (start 268.4 124.21) (end 267.4 124.21) (width 0.2) (layer "F.Cu") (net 2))
 (segment (start 266.9 126.11) (end 266.9 125.41) (width 0.2) (layer "F.Cu") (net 2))
 (segment (start 266.9 124.61) (end 266.9 124.565696) (width 0.2) (layer "F.Cu") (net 2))
 (segment (start 266.9 124.61) (end 267.35 124.16) (width 0.2) (layer "F.Cu") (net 2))
 (segment (start 266.9 124.565696) (end 266.444306 124.110002) (width 0.2) (layer "F.Cu") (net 2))
 (segment (start 267.4 124.21) (end 267.35 124.16) (width 0.2) (layer "F.Cu") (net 2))
 (via (at 267.399998 125.001386) (size 0.8) (drill 0.4) (layers "F.Cu" "B.Cu") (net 2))
 (via (at 266.400002 125.09857) (size 0.8) (drill 0.4) (layers "F.Cu" "B.Cu") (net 2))
 (via (at 267.35 124.16) (size 0.8) (drill 0.4) (layers "F.Cu" "B.Cu") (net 2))
 (via (at 266.444306 124.110002) (size 0.8) (drill 0.4) (layers "F.Cu" "B.Cu") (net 2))
 (segment (start 266.9 121.28) (end 266.9 123.11) (width 0.2) (layer "F.Cu") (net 4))
 (segment (start 264.15 116.96) (end 263.15 117.96) (width 0.2) (layer "F.Cu") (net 4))
 (segment (start 268.54 117.17) (end 269.55 116.16) (width 0.6) (layer "F.Cu") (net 4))
 (segment (start 268.54 118.07) (end 268.54 117.17) (width 0.6) (layer "F.Cu") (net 4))
 (segment (start 269.55 116.16) (end 273.15 116.16) (width 0.6) (layer "F.Cu") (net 4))
 (segment (start 268.54 118.07) (end 266.77 119.84) (width 0.2) (layer "F.Cu") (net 4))
 (segment (start 266.77 119.84) (end 266.77 121.15) (width 0.2) (layer "F.Cu") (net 4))
 (segment (start 267.43 116.96) (end 264.15 116.96) (width 0.2) (layer "F.Cu") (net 4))
 (segment (start 268.54 118.07) (end 267.43 116.96) (width 0.2) (layer "F.Cu") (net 4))
 (segment (start 263.15 117.96) (end 263.15 120.16) (width 0.2) (layer "F.Cu") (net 4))
 (segment (start 266.77 121.15) (end 266.9 121.28) (width 0.2) (layer "F.Cu") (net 4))
 (segment (start 268.4 124.61) (end 271.12 124.61) (width 0.2) (layer "F.Cu") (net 19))
 (segment (start 271.12 124.61) (end 271.15 124.58) (width 0.2) (layer "F.Cu") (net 19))
 (segment (start 268.95 125.96) (end 268.95 127.96) (width 0.2) (layer "F.Cu") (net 17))
 (segment (start 268.4 125.41) (end 268.95 125.96) (width 0.2) (layer "F.Cu") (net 17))
 (segment (start 269.25 129.46) (end 268.35 128.56) (width 0.2) (layer "F.Cu") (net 17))
 (segment (start 270.15 129.46) (end 269.25 129.46) (width 0.2) (layer "F.Cu") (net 17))
 (segment (start 268.95 127.96) (end 268.35 128.56) (width 0.2) (layer "F.Cu") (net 17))
 (segment (start 265.4 124.21) (end 264.26 124.21) (width 0.2) (layer "F.Cu") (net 12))
 (segment (start 263.15 123.1) (end 263.15 121.58) (width 0.2) (layer "F.Cu") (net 12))
 (segment (start 264.26 124.21) (end 263.15 123.1) (width 0.2) (layer "F.Cu") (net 12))
 (segment (start 271.7 129.51) (end 271.75 129.46) (width 0.2) (layer "F.Cu") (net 10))
 (segment (start 271.7 132.36) (end 271.7 129.51) (width 0.2) (layer "F.Cu") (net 10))
 (segment (start 272.35 133.36) (end 272.95 132.76) (width 0.2) (layer "F.Cu") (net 27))
 (segment (start 266.8 133.01) (end 267.15 133.36) (width 0.2) (layer "F.Cu") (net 27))
 (segment (start 267.15 133.36) (end 272.35 133.36) (width 0.2) (layer "F.Cu") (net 27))
 (segment (start 272.95 127.16) (end 272.45 126.66) (width 0.2) (layer "F.Cu") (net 27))
 (segment (start 272.45 126.66) (end 271.75 126.66) (width 0.2) (layer "F.Cu") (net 27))
 (segment (start 272.95 132.76) (end 272.95 127.16) (width 0.2) (layer "F.Cu") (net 27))
 (segment (start 266.8 132.36) (end 266.8 133.01) (width 0.2) (layer "F.Cu") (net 27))
 (segment (start 269.1 125.01) (end 270.15 126.06) (width 0.2) (layer "F.Cu") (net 18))
 (segment (start 270.15 126.06) (end 270.15 126.66) (width 0.2) (layer "F.Cu") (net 18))
 (segment (start 268.4 125.01) (end 269.1 125.01) (width 0.2) (layer "F.Cu") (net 18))
 (segment (start 266.1 122.11) (end 265.35 121.36) (width 0.2) (layer "F.Cu") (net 8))
 (segment (start 266.1 123.11) (end 266.1 122.11) (width 0.2) (layer "F.Cu") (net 8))
 (segment (start 267.7 123.11) (end 267.7 122.01) (width 0.2) (layer "F.Cu") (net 1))
 (segment (start 267.7 122.01) (end 268.55 121.16) (width 0.2) (layer "F.Cu") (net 1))
 (segment (start 263.2 124.61) (end 265.4 124.61) (width 0.2) (layer "F.Cu") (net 13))
 (segment (start 261.75 123.16) (end 263.2 124.61) (width 0.2) (layer "F.Cu") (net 13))
 (segment (start 261.75 125) (end 261.76 125.01) (width 0.2) (layer "F.Cu") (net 5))
 (segment (start 261.76 125.01) (end 265.4 125.01) (width 0.2) (layer "F.Cu") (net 5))
 (segment (start 261.75 126.84) (end 263.07 126.84) (width 0.2) (layer "F.Cu") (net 14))
 (segment (start 263.07 126.84) (end 264.5 125.41) (width 0.2) (layer "F.Cu") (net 14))
 (segment (start 264.5 125.41) (end 265.4 125.41) (width 0.2) (layer "F.Cu") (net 14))
 (segment (start 261.27 127.96) (end 262.35 127.96) (width 0.2) (layer "F.Cu") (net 15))
 (segment (start 264.85 127.36) (end 266.1 126.11) (width 0.2) (layer "F.Cu") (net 15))
 (segment (start 262.35 127.96) (end 262.95 127.36) (width 0.2) (layer "F.Cu") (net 15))
 (segment (start 262.95 127.36) (end 264.85 127.36) (width 0.2) (layer "F.Cu") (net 15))
 (segment (start 260.27 128.96) (end 261.27 127.96) (width 0.2) (layer "F.Cu") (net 15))
 (segment (start 265.295 128.015) (end 266.5 126.81) (width 0.2) (layer "F.Cu") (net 9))
 (segment (start 263.055 128.015) (end 265.295 128.015) (width 0.2) (layer "F.Cu") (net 9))
 (segment (start 262.11 128.96) (end 263.055 128.015) (width 0.2) (layer "F.Cu") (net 9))
 (segment (start 266.5 126.81) (end 266.5 126.11) (width 0.2) (layer "F.Cu") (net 9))
 (segment (start 267.7 126.81) (end 267.7 126.11) (width 0.2) (layer "F.Cu") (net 16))
 (segment (start 263.95 128.96) (end 265.55 128.96) (width 0.2) (layer "F.Cu") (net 16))
 (segment (start 265.55 128.96) (end 267.7 126.81) (width 0.2) (layer "F.Cu") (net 16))
 (segment (start 264.35 122.56) (end 264.35 122.96) (width 0.2) (layer "F.Cu") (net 11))
 (segment (start 264.35 122.96) (end 264.35 123.152894) (width 0.4) (layer "F.Cu") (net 11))
 (segment (start 264.897106 123.7) (end 264.91 123.7) (width 0.4) (layer "F.Cu") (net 11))
 (segment (start 264.35 123.152894) (end 264.897106 123.7) (width 0.4) (layer "F.Cu") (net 11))
 (segment (start 109.38 119.95) (end 110.13 120.7) (width 0.2) (layer "F.Cu") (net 11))
 (segment (start 108.23 119.95) (end 109.38 119.95) (width 0.2) (layer "F.Cu") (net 11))
 (segment (start 264.91 123.7) (end 265.02 123.81) (width 0.2) (layer "F.Cu") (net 11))
 (segment (start 265.02 123.81) (end 265.4 123.81) (width 0.2) (layer "F.Cu") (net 11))
 (via (at 110.13 120.7) (size 0.8) (drill 0.4) (layers "F.Cu" "B.Cu") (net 11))
 (via (at 264.35 122.56) (size 0.8) (drill 0.4) (layers "F.Cu" "B.Cu") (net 11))
 (segment (start 268.9 123.81) (end 269.05 123.66) (width 0.2) (layer "F.Cu") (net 20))
 (segment (start 268.4 123.81) (end 268.9 123.81) (width 0.2) (layer "F.Cu") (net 20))
 (segment (start 269.05 123.66) (end 269.75 122.96) (width 0.4) (layer "F.Cu") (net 20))
 (segment (start 108.23 117.45) (end 109.18 117.45) (width 0.2) (layer "F.Cu") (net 20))
 (segment (start 109.18 117.45) (end 110.13 116.5) (width 0.2) (layer "F.Cu") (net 20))
 (via (at 269.75 122.96) (size 0.8) (drill 0.4) (layers "F.Cu" "B.Cu") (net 20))
 (via (at 110.13 116.5) (size 0.8) (drill 0.4) (layers "F.Cu" "B.Cu") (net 20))
 (segment (start 272.13 118.88) (end 271.51 119.5) (width 0.4) (layer "F.Cu") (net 21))
 (segment (start 267.3 120.385) (end 267.3 123.11) (width 0.2) (layer "F.Cu") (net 21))
 (segment (start 108.23 118.7) (end 110.13 118.7) (width 0.2) (layer "F.Cu") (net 21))
 (segment (start 268.185 119.5) (end 267.3 120.385) (width 0.4) (layer "F.Cu") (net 21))
 (segment (start 271.51 119.5) (end 268.185 119.5) (width 0.4) (layer "F.Cu") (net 21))
 (via (at 272.13 118.88) (size 0.8) (drill 0.4) (layers "F.Cu" "B.Cu") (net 21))
 (via (at 110.13 118.7) (size 0.8) (drill 0.4) (layers "F.Cu" "B.Cu") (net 21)))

